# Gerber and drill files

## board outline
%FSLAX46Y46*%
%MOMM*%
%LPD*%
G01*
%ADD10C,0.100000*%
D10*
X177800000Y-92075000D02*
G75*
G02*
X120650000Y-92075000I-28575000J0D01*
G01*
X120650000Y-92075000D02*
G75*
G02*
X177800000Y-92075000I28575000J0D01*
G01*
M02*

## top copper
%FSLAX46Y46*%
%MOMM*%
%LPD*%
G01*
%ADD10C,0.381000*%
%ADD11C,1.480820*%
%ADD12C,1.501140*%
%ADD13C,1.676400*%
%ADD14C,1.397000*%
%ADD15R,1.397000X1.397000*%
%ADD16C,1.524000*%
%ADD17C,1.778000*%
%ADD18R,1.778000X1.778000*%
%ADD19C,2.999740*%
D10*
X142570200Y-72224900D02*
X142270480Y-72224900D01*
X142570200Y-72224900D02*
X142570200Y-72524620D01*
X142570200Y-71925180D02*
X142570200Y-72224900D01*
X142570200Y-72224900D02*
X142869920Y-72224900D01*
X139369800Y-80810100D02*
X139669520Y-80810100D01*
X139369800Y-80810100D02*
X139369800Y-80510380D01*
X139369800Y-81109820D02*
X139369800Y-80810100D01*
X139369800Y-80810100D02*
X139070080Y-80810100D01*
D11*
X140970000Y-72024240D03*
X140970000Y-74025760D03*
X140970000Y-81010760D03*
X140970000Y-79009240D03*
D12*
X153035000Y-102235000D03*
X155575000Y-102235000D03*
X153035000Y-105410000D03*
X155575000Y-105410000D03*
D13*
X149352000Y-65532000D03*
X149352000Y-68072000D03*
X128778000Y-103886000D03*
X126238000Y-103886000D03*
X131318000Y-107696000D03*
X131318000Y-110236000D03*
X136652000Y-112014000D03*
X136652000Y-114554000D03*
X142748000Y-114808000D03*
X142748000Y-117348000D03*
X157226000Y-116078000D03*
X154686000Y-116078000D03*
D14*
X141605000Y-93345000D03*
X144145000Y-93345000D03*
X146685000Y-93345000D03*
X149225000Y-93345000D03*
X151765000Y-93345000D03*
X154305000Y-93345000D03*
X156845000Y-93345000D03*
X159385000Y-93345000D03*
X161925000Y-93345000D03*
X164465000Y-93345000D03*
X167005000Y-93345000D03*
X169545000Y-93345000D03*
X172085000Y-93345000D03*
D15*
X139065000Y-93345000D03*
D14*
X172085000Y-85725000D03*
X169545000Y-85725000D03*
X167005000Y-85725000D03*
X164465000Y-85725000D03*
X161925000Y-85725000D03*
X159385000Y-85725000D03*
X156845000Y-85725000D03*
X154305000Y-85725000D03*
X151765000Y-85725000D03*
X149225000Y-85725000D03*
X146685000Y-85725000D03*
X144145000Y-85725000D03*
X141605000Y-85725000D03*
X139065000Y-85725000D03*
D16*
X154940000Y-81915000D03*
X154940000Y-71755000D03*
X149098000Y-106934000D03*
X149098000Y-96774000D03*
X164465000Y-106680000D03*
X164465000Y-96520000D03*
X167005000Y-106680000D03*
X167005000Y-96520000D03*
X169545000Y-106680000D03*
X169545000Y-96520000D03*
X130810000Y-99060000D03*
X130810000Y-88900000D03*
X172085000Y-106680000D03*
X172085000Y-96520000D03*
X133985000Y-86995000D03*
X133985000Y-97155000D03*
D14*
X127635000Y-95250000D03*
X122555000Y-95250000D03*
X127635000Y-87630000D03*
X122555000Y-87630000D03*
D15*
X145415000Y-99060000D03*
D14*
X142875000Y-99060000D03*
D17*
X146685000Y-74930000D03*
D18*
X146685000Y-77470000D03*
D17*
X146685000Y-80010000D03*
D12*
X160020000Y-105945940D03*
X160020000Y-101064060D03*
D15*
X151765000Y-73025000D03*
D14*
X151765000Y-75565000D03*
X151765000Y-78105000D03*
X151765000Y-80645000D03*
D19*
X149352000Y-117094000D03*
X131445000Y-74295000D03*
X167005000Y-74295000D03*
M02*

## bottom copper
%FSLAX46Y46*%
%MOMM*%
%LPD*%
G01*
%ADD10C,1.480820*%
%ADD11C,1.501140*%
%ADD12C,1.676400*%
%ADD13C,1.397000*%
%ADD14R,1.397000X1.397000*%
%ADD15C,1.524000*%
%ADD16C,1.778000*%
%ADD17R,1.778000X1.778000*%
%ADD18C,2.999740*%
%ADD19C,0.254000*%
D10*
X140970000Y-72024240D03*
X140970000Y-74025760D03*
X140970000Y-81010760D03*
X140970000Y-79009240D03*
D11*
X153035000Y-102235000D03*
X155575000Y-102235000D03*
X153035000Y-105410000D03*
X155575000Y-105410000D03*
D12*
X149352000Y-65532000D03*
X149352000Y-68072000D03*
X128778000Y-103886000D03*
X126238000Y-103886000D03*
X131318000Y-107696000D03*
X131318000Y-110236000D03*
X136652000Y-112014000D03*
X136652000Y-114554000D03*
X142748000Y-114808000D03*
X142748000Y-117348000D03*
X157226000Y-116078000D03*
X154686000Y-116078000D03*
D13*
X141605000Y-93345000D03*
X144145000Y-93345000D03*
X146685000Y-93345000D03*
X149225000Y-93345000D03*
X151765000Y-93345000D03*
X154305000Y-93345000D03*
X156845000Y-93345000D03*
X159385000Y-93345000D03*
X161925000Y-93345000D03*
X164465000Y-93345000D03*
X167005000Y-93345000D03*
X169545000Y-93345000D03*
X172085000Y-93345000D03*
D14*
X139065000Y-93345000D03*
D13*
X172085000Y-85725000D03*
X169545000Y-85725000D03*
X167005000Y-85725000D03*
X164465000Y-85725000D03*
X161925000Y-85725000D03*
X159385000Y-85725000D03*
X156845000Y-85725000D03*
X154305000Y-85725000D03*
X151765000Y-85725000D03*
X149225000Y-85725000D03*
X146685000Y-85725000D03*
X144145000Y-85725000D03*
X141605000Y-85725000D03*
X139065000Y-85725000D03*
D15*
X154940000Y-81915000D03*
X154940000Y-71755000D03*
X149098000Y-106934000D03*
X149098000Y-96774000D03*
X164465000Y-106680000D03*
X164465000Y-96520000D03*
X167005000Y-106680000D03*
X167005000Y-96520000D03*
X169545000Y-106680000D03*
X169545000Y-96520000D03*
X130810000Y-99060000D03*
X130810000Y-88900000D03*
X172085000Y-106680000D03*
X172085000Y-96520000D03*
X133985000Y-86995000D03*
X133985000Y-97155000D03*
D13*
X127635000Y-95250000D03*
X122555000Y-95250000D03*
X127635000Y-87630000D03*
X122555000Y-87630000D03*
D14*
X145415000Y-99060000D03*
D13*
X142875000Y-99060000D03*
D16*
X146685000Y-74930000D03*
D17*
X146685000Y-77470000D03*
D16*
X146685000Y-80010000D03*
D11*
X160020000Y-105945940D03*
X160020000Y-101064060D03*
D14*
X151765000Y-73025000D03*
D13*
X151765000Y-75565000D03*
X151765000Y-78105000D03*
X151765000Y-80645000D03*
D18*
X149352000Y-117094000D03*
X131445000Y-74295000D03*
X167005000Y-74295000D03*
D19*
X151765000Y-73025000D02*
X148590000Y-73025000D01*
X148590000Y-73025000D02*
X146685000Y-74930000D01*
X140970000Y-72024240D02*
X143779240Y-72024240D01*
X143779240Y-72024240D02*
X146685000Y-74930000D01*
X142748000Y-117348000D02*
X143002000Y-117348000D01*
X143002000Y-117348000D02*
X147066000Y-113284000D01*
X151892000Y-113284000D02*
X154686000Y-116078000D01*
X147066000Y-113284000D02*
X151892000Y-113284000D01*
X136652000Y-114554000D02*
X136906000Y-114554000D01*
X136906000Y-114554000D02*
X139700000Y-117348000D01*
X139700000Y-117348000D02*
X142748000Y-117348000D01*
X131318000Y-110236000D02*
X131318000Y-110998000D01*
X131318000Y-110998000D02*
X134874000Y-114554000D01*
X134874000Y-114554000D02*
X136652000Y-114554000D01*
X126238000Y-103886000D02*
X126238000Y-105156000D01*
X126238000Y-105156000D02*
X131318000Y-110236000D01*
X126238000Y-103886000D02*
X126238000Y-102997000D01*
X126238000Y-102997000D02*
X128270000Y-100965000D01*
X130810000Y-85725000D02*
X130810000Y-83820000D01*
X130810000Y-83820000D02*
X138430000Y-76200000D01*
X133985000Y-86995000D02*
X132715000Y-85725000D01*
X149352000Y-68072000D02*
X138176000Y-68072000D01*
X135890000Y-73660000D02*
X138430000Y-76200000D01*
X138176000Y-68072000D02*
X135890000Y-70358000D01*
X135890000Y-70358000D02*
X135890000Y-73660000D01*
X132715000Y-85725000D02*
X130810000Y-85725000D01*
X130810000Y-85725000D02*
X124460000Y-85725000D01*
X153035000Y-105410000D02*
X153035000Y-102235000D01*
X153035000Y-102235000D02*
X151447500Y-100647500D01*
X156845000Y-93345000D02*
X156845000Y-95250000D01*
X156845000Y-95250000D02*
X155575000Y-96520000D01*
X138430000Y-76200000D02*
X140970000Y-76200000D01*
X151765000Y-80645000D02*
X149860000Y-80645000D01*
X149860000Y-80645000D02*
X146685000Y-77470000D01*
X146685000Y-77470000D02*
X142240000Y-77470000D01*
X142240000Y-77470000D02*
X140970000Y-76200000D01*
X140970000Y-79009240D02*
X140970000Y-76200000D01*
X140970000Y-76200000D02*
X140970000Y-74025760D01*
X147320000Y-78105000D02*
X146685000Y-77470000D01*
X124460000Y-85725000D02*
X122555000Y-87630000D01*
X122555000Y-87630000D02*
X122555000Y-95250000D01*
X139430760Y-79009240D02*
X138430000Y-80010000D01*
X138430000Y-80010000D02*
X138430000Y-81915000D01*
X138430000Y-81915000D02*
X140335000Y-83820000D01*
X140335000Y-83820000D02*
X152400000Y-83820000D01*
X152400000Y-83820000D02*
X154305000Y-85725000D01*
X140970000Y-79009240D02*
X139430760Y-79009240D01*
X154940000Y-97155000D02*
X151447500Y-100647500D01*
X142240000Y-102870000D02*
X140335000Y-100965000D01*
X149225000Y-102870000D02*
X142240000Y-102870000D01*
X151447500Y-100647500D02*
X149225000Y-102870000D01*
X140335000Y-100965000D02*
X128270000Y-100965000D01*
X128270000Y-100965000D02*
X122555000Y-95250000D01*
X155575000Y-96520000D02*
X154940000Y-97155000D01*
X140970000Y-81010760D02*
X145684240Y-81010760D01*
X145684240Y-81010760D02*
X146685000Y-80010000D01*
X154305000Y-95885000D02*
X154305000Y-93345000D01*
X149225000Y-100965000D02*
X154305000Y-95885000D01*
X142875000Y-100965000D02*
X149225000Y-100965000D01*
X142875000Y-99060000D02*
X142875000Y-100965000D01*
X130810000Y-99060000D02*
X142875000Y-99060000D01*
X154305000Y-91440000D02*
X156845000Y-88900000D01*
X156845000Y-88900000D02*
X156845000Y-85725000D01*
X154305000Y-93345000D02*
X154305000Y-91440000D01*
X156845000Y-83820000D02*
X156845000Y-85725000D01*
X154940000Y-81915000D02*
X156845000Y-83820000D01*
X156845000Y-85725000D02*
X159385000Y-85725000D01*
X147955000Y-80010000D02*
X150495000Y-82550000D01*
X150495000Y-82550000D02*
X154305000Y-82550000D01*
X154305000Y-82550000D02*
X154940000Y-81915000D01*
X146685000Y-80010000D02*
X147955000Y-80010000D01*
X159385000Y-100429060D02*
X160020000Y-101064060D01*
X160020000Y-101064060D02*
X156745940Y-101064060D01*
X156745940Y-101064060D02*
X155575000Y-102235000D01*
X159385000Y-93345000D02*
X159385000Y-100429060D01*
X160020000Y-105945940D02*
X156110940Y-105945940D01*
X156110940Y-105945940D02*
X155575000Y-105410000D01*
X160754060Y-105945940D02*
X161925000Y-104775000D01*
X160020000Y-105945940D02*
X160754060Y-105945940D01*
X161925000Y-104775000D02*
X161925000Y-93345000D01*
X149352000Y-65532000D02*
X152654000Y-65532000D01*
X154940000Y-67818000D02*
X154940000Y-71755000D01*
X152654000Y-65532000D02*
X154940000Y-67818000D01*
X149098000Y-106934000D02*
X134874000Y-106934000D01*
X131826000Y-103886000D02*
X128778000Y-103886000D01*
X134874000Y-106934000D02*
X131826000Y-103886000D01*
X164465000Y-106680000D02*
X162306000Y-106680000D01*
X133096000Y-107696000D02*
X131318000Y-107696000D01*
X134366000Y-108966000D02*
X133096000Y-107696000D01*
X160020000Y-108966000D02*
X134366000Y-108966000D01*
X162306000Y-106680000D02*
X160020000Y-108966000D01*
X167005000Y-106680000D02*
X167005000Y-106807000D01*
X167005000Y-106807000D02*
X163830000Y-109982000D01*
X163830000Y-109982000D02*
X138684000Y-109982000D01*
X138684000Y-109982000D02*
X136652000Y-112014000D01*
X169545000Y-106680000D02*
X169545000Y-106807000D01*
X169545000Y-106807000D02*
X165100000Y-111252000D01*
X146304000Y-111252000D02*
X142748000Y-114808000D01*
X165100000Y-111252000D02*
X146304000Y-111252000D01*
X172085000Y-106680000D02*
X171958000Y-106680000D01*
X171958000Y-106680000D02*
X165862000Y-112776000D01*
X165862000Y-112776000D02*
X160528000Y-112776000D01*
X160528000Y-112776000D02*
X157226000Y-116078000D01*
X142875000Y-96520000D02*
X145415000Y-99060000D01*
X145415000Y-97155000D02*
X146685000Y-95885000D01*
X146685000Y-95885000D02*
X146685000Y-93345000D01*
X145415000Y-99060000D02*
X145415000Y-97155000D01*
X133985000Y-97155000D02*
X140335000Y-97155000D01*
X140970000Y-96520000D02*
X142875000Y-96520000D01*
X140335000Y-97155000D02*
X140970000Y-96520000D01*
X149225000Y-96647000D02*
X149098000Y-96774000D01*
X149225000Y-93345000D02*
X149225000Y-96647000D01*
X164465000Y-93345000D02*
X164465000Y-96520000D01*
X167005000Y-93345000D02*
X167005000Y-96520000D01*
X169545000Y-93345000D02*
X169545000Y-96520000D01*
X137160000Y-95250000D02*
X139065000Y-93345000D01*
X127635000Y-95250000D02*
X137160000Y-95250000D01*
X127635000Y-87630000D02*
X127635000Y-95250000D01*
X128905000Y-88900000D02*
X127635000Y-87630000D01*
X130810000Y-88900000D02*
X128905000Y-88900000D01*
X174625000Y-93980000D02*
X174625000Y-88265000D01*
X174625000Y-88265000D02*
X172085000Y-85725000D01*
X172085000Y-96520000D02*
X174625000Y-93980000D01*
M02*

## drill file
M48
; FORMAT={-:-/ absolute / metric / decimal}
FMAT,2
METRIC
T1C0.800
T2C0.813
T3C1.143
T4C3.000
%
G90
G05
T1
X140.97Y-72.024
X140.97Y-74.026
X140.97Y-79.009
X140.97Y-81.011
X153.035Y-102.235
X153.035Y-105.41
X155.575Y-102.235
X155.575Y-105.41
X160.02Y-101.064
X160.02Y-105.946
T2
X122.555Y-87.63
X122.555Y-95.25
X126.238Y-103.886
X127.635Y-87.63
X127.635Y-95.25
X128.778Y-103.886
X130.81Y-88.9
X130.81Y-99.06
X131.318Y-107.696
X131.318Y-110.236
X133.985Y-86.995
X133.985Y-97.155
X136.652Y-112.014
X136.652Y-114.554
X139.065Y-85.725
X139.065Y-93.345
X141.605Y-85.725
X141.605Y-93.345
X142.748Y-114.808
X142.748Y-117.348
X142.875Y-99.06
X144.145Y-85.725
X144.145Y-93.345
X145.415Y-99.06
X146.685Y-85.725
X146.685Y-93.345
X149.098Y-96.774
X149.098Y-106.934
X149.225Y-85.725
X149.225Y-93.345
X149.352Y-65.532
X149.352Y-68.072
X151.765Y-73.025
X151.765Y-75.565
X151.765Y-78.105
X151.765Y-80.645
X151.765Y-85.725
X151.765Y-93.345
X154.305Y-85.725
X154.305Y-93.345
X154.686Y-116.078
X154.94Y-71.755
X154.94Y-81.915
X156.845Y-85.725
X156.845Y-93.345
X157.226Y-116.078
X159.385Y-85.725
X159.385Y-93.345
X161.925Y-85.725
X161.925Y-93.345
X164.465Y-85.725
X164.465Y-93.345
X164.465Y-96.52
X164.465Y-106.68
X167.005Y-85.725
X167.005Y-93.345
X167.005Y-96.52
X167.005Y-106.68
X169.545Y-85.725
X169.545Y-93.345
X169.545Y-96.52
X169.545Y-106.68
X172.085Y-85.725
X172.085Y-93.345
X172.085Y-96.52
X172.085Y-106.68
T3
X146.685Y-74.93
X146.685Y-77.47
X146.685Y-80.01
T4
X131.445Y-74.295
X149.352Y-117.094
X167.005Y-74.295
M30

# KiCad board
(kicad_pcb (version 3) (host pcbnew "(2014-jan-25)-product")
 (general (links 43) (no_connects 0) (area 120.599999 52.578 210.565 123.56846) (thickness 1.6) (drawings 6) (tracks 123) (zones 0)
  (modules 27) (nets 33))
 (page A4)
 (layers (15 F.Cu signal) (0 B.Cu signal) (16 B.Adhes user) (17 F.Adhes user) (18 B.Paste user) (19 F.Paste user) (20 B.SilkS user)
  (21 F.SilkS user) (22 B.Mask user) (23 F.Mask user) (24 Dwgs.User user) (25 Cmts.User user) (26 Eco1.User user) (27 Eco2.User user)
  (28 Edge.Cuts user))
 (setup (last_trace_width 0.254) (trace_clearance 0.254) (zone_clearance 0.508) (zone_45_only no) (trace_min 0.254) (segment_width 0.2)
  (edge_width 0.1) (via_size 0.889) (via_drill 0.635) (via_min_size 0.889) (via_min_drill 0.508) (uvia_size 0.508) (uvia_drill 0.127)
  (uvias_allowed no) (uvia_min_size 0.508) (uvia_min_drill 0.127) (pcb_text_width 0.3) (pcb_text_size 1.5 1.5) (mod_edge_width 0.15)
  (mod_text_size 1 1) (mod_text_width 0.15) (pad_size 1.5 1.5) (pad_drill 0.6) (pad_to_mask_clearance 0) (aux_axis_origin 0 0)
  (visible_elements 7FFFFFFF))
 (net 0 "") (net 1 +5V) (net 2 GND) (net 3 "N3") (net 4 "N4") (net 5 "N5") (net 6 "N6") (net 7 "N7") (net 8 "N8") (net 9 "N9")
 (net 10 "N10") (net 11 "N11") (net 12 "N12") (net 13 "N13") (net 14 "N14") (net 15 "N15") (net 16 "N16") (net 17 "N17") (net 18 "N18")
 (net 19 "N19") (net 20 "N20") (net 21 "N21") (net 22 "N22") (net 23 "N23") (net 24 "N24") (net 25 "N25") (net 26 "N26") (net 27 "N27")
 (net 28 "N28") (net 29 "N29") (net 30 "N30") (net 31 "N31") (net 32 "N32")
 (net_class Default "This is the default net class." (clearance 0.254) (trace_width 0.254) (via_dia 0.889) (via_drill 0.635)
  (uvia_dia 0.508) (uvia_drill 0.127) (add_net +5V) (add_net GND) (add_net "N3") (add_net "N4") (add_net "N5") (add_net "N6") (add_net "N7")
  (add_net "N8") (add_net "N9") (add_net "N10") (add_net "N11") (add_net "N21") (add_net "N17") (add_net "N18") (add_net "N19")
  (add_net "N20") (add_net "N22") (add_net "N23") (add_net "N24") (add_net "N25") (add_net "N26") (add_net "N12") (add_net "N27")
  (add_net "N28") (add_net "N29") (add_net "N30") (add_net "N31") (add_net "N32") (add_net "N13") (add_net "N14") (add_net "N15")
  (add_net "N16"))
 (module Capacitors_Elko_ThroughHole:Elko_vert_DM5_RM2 (layer F.Cu) (at 140.97 73.025 270)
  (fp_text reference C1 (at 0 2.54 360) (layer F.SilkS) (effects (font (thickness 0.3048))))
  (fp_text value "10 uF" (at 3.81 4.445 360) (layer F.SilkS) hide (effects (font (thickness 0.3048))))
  (fp_line (start -0.8001 -1.6002) (end -0.8001 -1.30048) (layer F.Cu) (width 0.381))
  (fp_line (start -0.8001 -1.6002) (end -0.50038 -1.6002) (layer F.Cu) (width 0.381))
  (fp_line (start -1.09982 -1.6002) (end -0.8001 -1.6002) (layer F.Cu) (width 0.381))
  (fp_line (start -0.8001 -1.6002) (end -0.8001 -1.89992) (layer F.Cu) (width 0.381))
  (pad 1 thru_hole circle (at -1.00076 0 270) (size 1.48082 1.48082) (drill 0.8001) (layers *.Cu *.Mask F.SilkS) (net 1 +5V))
  (pad 2 thru_hole circle (at 1.00076 0 270) (size 1.48082 1.48082) (drill 0.8001) (layers *.Cu *.Mask F.SilkS) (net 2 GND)))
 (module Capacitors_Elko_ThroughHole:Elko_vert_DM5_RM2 (layer F.Cu) (at 140.97 80.01 90)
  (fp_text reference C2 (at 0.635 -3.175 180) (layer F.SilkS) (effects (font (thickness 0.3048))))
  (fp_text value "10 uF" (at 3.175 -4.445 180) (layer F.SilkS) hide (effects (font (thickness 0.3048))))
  (fp_line (start -0.8001 -1.6002) (end -0.8001 -1.30048) (layer F.Cu) (width 0.381))
  (fp_line (start -0.8001 -1.6002) (end -0.50038 -1.6002) (layer F.Cu) (width 0.381))
  (fp_line (start -1.09982 -1.6002) (end -0.8001 -1.6002) (layer F.Cu) (width 0.381))
  (fp_line (start -0.8001 -1.6002) (end -0.8001 -1.89992) (layer F.Cu) (width 0.381))
  (pad 1 thru_hole circle (at -1.00076 0 90) (size 1.48082 1.48082) (drill 0.8001) (layers *.Cu *.Mask F.SilkS) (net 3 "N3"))
  (pad 2 thru_hole circle (at 1.00076 0 90) (size 1.48082 1.48082) (drill 0.8001) (layers *.Cu *.Mask F.SilkS) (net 2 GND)))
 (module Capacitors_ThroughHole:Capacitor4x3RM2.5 (layer F.Cu) (at 153.035 102.235)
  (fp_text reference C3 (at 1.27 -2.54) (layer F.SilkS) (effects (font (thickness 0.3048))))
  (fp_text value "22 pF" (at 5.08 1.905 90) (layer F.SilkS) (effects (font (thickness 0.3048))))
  (pad 1 thru_hole circle (at 0 0) (size 1.50114 1.50114) (drill 0.8001) (layers *.Cu *.Mask F.SilkS) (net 2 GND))
  (pad 2 thru_hole circle (at 2.54 0) (size 1.50114 1.50114) (drill 0.8001) (layers *.Cu *.Mask F.SilkS) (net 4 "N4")))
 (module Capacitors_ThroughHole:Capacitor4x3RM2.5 (layer F.Cu) (at 153.035 105.41)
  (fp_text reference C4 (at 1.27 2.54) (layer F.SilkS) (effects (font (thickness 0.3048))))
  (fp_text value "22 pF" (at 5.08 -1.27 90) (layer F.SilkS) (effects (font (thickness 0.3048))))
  (pad 1 thru_hole circle (at 0 0) (size 1.50114 1.50114) (drill 0.8001) (layers *.Cu *.Mask F.SilkS) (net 2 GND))
  (pad 2 thru_hole circle (at 2.54 0) (size 1.50114 1.50114) (drill 0.8001) (layers *.Cu *.Mask F.SilkS) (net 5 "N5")))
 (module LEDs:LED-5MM (layer F.Cu) (at 149.352 66.802 270)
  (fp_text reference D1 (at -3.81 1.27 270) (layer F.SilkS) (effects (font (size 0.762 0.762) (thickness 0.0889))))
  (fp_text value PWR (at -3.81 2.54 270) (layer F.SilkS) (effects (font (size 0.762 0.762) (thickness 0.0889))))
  (pad 1 thru_hole circle (at -1.27 0 270) (size 1.6764 1.6764) (drill 0.8128) (layers *.Cu *.Mask F.SilkS) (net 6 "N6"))
  (pad 2 thru_hole circle (at 1.27 0 270) (size 1.6764 1.6764) (drill 0.8128) (layers *.Cu *.Mask F.SilkS) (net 2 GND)))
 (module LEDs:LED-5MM (layer F.Cu) (at 127.508 103.886 180)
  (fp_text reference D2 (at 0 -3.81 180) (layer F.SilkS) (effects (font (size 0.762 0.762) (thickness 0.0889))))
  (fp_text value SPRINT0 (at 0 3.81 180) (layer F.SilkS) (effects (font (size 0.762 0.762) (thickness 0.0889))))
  (pad 1 thru_hole circle (at -1.27 0 180) (size 1.6764 1.6764) (drill 0.8128) (layers *.Cu *.Mask F.SilkS) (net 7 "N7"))
  (pad 2 thru_hole circle (at 1.27 0 180) (size 1.6764 1.6764) (drill 0.8128) (layers *.Cu *.Mask F.SilkS) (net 2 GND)))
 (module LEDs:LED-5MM (layer F.Cu) (at 131.318 108.966 270)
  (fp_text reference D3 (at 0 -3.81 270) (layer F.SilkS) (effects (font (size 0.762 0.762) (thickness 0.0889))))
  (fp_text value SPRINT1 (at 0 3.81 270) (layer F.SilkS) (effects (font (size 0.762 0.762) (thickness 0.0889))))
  (pad 1 thru_hole circle (at -1.27 0 270) (size 1.6764 1.6764) (drill 0.8128) (layers *.Cu *.Mask F.SilkS) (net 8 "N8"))
  (pad 2 thru_hole circle (at 1.27 0 270) (size 1.6764 1.6764) (drill 0.8128) (layers *.Cu *.Mask F.SilkS) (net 2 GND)))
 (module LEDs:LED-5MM (layer F.Cu) (at 136.652 113.284 270)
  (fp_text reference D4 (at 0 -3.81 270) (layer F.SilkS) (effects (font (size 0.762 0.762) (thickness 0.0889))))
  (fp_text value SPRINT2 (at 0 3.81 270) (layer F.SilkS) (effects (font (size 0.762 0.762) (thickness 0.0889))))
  (pad 1 thru_hole circle (at -1.27 0 270) (size 1.6764 1.6764) (drill 0.8128) (layers *.Cu *.Mask F.SilkS) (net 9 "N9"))
  (pad 2 thru_hole circle (at 1.27 0 270) (size 1.6764 1.6764) (drill 0.8128) (layers *.Cu *.Mask F.SilkS) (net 2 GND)))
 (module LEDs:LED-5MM (layer F.Cu) (at 142.748 116.078 270)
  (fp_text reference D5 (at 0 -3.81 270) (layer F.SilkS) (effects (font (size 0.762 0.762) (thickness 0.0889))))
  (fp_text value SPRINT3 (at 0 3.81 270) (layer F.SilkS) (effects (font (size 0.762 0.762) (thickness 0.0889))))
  (pad 1 thru_hole circle (at -1.27 0 270) (size 1.6764 1.6764) (drill 0.8128) (layers *.Cu *.Mask F.SilkS) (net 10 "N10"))
  (pad 2 thru_hole circle (at 1.27 0 270) (size 1.6764 1.6764) (drill 0.8128) (layers *.Cu *.Mask F.SilkS) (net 2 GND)))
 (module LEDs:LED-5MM (layer F.Cu) (at 155.956 116.078 180)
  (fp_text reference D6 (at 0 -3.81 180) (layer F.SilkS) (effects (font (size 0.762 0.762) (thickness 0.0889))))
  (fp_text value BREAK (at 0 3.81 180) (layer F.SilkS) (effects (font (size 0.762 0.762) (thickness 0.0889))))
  (pad 1 thru_hole circle (at -1.27 0 180) (size 1.6764 1.6764) (drill 0.8128) (layers *.Cu *.Mask F.SilkS) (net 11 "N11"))
  (pad 2 thru_hole circle (at 1.27 0 180) (size 1.6764 1.6764) (drill 0.8128) (layers *.Cu *.Mask F.SilkS) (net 2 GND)))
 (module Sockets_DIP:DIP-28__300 (layer F.Cu) (at 155.575 89.535)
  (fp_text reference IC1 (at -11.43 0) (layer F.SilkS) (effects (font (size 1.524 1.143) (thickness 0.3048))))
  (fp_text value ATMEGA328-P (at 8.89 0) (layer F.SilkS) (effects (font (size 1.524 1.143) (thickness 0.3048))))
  (pad 2 thru_hole circle (at -13.97 3.81) (size 1.397 1.397) (drill 0.8128) (layers *.Cu *.Mask F.SilkS) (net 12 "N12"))
  (pad 3 thru_hole circle (at -11.43 3.81) (size 1.397 1.397) (drill 0.8128) (layers *.Cu *.Mask F.SilkS) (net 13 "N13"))
  (pad 4 thru_hole circle (at -8.89 3.81) (size 1.397 1.397) (drill 0.8128) (layers *.Cu *.Mask F.SilkS) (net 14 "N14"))
  (pad 5 thru_hole circle (at -6.35 3.81) (size 1.397 1.397) (drill 0.8128) (layers *.Cu *.Mask F.SilkS) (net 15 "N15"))
  (pad 6 thru_hole circle (at -3.81 3.81) (size 1.397 1.397) (drill 0.8128) (layers *.Cu *.Mask F.SilkS) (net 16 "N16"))
  (pad 7 thru_hole circle (at -1.27 3.81) (size 1.397 1.397) (drill 0.8128) (layers *.Cu *.Mask F.SilkS) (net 3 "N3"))
  (pad 8 thru_hole circle (at 1.27 3.81) (size 1.397 1.397) (drill 0.8128) (layers *.Cu *.Mask F.SilkS) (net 2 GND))
  (pad 9 thru_hole circle (at 3.81 3.81) (size 1.397 1.397) (drill 0.8128) (layers *.Cu *.Mask F.SilkS) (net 4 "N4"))
  (pad 10 thru_hole circle (at 6.35 3.81) (size 1.397 1.397) (drill 0.8128) (layers *.Cu *.Mask F.SilkS) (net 5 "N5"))
  (pad 11 thru_hole circle (at 8.89 3.81) (size 1.397 1.397) (drill 0.8128) (layers *.Cu *.Mask F.SilkS) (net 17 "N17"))
  (pad 12 thru_hole circle (at 11.43 3.81) (size 1.397 1.397) (drill 0.8128) (layers *.Cu *.Mask F.SilkS) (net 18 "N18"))
  (pad 13 thru_hole circle (at 13.97 3.81) (size 1.397 1.397) (drill 0.8128) (layers *.Cu *.Mask F.SilkS) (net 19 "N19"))
  (pad 14 thru_hole circle (at 16.51 3.81) (size 1.397 1.397) (drill 0.8128) (layers *.Cu *.Mask F.SilkS) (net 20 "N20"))
  (pad 1 thru_hole rect (at -16.51 3.81) (size 1.397 1.397) (drill 0.8128) (layers *.Cu *.Mask F.SilkS) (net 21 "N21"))
  (pad 15 thru_hole circle (at 16.51 -3.81) (size 1.397 1.397) (drill 0.8128) (layers *.Cu *.Mask F.SilkS) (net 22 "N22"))
  (pad 16 thru_hole circle (at 13.97 -3.81) (size 1.397 1.397) (drill 0.8128) (layers *.Cu *.Mask F.SilkS) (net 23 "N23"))
  (pad 17 thru_hole circle (at 11.43 -3.81) (size 1.397 1.397) (drill 0.8128) (layers *.Cu *.Mask F.SilkS) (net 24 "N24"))
  (pad 18 thru_hole circle (at 8.89 -3.81) (size 1.397 1.397) (drill 0.8128) (layers *.Cu *.Mask F.SilkS) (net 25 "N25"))
  (pad 19 thru_hole circle (at 6.35 -3.81) (size 1.397 1.397) (drill 0.8128) (layers *.Cu *.Mask F.SilkS) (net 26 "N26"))
  (pad 20 thru_hole circle (at 3.81 -3.81) (size 1.397 1.397) (drill 0.8128) (layers *.Cu *.Mask F.SilkS) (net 3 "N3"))
  (pad 21 thru_hole circle (at 1.27 -3.81) (size 1.397 1.397) (drill 0.8128) (layers *.Cu *.Mask F.SilkS) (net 3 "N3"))
  (pad 22 thru_hole circle (at -1.27 -3.81) (size 1.397 1.397) (drill 0.8128) (layers *.Cu *.Mask F.SilkS) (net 2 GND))
  (pad 23 thru_hole circle (at -3.81 -3.81) (size 1.397 1.397) (drill 0.8128) (layers *.Cu *.Mask F.SilkS) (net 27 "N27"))
  (pad 24 thru_hole circle (at -6.35 -3.81) (size 1.397 1.397) (drill 0.8128) (layers *.Cu *.Mask F.SilkS) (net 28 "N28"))
  (pad 25 thru_hole circle (at -8.89 -3.81) (size 1.397 1.397) (drill 0.8128) (layers *.Cu *.Mask F.SilkS) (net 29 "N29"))
  (pad 26 thru_hole circle (at -11.43 -3.81) (size 1.397 1.397) (drill 0.8128) (layers *.Cu *.Mask F.SilkS) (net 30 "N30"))
  (pad 27 thru_hole circle (at -13.97 -3.81) (size 1.397 1.397) (drill 0.8128) (layers *.Cu *.Mask F.SilkS) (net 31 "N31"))
  (pad 28 thru_hole circle (at -16.51 -3.81) (size 1.397 1.397) (drill 0.8128) (layers *.Cu *.Mask F.SilkS) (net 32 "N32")))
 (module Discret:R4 (layer F.Cu) (at 154.94 76.835 90) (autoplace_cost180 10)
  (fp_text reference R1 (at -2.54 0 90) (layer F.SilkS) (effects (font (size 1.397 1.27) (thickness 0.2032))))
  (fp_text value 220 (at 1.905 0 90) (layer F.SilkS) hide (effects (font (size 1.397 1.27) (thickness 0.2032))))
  (pad 1 thru_hole circle (at -5.08 0 90) (size 1.524 1.524) (drill 0.8128) (layers *.Cu *.Mask F.SilkS) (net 3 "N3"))
  (pad 2 thru_hole circle (at 5.08 0 90) (size 1.524 1.524) (drill 0.8128) (layers *.Cu *.Mask F.SilkS) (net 6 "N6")))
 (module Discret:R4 (layer F.Cu) (at 149.098 101.854 90) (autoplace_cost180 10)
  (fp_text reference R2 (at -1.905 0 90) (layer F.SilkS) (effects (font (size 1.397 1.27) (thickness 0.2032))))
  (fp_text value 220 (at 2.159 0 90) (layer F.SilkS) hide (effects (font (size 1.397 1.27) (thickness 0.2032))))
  (pad 1 thru_hole circle (at -5.08 0 90) (size 1.524 1.524) (drill 0.8128) (layers *.Cu *.Mask F.SilkS) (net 7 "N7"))
  (pad 2 thru_hole circle (at 5.08 0 90) (size 1.524 1.524) (drill 0.8128) (layers *.Cu *.Mask F.SilkS) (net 15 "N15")))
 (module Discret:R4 (layer F.Cu) (at 164.465 101.6 90) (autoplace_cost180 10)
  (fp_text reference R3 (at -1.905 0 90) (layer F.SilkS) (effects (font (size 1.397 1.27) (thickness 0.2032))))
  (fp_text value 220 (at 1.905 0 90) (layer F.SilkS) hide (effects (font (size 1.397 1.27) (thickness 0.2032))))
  (pad 1 thru_hole circle (at -5.08 0 90) (size 1.524 1.524) (drill 0.8128) (layers *.Cu *.Mask F.SilkS) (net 8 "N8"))
  (pad 2 thru_hole circle (at 5.08 0 90) (size 1.524 1.524) (drill 0.8128) (layers *.Cu *.Mask F.SilkS) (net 17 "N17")))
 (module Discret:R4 (layer F.Cu) (at 167.005 101.6 90) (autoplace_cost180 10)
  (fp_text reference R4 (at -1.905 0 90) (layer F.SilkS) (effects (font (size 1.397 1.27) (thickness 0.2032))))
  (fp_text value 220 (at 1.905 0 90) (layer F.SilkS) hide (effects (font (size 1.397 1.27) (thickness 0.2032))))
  (pad 1 thru_hole circle (at -5.08 0 90) (size 1.524 1.524) (drill 0.8128) (layers *.Cu *.Mask F.SilkS) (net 9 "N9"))
  (pad 2 thru_hole circle (at 5.08 0 90) (size 1.524 1.524) (drill 0.8128) (layers *.Cu *.Mask F.SilkS) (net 18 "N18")))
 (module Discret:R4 (layer F.Cu) (at 169.545 101.6 90) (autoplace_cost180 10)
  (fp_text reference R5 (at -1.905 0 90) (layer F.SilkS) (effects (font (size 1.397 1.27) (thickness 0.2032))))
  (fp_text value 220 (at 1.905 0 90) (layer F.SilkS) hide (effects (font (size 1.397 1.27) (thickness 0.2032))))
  (pad 1 thru_hole circle (at -5.08 0 90) (size 1.524 1.524) (drill 0.8128) (layers *.Cu *.Mask F.SilkS) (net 10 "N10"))
  (pad 2 thru_hole circle (at 5.08 0 90) (size 1.524 1.524) (drill 0.8128) (layers *.Cu *.Mask F.SilkS) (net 19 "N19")))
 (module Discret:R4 (layer F.Cu) (at 130.81 93.98 90) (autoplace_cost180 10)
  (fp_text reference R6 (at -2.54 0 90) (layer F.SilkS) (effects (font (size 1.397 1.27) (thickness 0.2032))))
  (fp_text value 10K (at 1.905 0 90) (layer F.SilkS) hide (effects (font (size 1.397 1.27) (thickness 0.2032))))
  (pad 1 thru_hole circle (at -5.08 0 90) (size 1.524 1.524) (drill 0.8128) (layers *.Cu *.Mask F.SilkS) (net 3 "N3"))
  (pad 2 thru_hole circle (at 5.08 0 90) (size 1.524 1.524) (drill 0.8128) (layers *.Cu *.Mask F.SilkS) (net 21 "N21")))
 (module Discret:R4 (layer F.Cu) (at 172.085 101.6 90) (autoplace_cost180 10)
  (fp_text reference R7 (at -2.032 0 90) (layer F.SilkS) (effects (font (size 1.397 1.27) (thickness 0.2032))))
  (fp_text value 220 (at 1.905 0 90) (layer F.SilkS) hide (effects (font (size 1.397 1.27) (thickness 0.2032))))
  (pad 1 thru_hole circle (at -5.08 0 90) (size 1.524 1.524) (drill 0.8128) (layers *.Cu *.Mask F.SilkS) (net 11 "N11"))
  (pad 2 thru_hole circle (at 5.08 0 90) (size 1.524 1.524) (drill 0.8128) (layers *.Cu *.Mask F.SilkS) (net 22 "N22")))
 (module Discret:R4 (layer F.Cu) (at 133.985 92.075 270) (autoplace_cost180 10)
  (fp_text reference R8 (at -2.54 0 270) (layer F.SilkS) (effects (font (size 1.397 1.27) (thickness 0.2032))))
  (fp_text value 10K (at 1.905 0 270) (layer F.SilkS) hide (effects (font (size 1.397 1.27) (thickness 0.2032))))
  (pad 1 thru_hole circle (at -5.08 0 270) (size 1.524 1.524) (drill 0.8128) (layers *.Cu *.Mask F.SilkS) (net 2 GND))
  (pad 2 thru_hole circle (at 5.08 0 270) (size 1.524 1.524) (drill 0.8128) (layers *.Cu *.Mask F.SilkS) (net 14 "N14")))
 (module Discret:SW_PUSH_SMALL (layer F.Cu) (at 125.095 91.44 270)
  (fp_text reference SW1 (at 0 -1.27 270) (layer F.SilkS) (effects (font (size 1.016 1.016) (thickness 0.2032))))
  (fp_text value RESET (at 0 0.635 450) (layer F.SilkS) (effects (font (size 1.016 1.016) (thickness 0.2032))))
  (pad 1 thru_hole circle (at 3.81 -2.54 270) (size 1.397 1.397) (drill 0.8128) (layers *.Cu *.Mask F.SilkS) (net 21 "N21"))
  (pad 2 thru_hole circle (at 3.81 2.54 270) (size 1.397 1.397) (drill 0.8128) (layers *.Cu *.Mask F.SilkS) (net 2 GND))
  (pad 1 thru_hole circle (at -3.81 -2.54 270) (size 1.397 1.397) (drill 0.8128) (layers *.Cu *.Mask F.SilkS) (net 21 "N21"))
  (pad 2 thru_hole circle (at -3.81 2.54 270) (size 1.397 1.397) (drill 0.8128) (layers *.Cu *.Mask F.SilkS) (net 2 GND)))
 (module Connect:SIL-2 (layer F.Cu) (at 144.145 99.06 180)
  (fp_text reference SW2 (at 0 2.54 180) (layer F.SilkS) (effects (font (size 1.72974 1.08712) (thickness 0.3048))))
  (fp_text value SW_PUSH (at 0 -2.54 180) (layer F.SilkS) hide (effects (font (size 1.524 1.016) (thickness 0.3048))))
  (pad 1 thru_hole rect (at -1.27 0 180) (size 1.397 1.397) (drill 0.8128) (layers *.Cu *.Mask F.SilkS) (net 14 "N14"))
  (pad 2 thru_hole circle (at 1.27 0 180) (size 1.397 1.397) (drill 0.8128) (layers *.Cu *.Mask F.SilkS) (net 3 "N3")))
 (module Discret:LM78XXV (layer F.Cu) (at 146.685 77.47)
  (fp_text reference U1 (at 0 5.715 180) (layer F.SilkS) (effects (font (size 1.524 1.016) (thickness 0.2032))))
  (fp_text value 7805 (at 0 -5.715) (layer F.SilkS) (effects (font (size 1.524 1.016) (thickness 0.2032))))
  (pad VI thru_hole circle (at 0 -2.54) (size 1.778 1.778) (drill 1.143) (layers *.Cu *.Mask F.SilkS) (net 1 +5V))
  (pad GND thru_hole rect (at 0 0) (size 1.778 1.778) (drill 1.143) (layers *.Cu *.Mask F.SilkS) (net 2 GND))
  (pad VO thru_hole circle (at 0 2.54) (size 1.778 1.778) (drill 1.143) (layers *.Cu *.Mask F.SilkS) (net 3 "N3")))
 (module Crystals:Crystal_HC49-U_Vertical (layer F.Cu) (at 160.02 103.505 90)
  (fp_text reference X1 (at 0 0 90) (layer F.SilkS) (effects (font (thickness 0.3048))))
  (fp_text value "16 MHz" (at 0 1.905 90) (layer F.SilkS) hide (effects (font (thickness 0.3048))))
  (pad 1 thru_hole circle (at -2.44094 0 90) (size 1.50114 1.50114) (drill 0.8001) (layers *.Cu *.Mask F.SilkS) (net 5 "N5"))
  (pad 2 thru_hole circle (at 2.44094 0 90) (size 1.50114 1.50114) (drill 0.8001) (layers *.Cu *.Mask F.SilkS) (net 4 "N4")))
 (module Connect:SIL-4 (layer F.Cu) (at 151.765 76.835 270)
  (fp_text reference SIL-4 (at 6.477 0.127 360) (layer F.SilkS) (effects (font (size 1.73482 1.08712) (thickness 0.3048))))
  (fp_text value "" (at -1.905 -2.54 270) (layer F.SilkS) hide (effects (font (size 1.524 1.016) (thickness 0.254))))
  (pad 1 thru_hole rect (at -3.81 0 270) (size 1.397 1.397) (drill 0.8128) (layers *.Cu *.Mask F.SilkS))
  (pad 2 thru_hole circle (at -1.27 0 270) (size 1.397 1.397) (drill 0.8128) (layers *.Cu *.Mask F.SilkS))
  (pad 3 thru_hole circle (at 1.27 0 270) (size 1.397 1.397) (drill 0.8128) (layers *.Cu *.Mask F.SilkS))
  (pad 4 thru_hole circle (at 3.81 0 270) (size 1.397 1.397) (drill 0.8128) (layers *.Cu *.Mask F.SilkS)))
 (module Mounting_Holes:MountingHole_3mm (layer F.Cu) (at 149.352 117.094)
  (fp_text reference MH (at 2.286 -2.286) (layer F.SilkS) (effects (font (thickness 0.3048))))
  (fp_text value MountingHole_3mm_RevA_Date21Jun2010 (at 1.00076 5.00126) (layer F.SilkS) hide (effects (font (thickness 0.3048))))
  (pad 1 thru_hole circle (at 0 0) (size 2.99974 2.99974) (drill 2.99974) (layers)))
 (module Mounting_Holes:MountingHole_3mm (layer F.Cu) (at 131.445 74.295)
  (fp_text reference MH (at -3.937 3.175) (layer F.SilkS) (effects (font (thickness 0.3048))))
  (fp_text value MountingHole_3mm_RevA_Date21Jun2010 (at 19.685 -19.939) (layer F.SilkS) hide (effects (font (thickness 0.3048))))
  (pad 1 thru_hole circle (at 0 0) (size 2.99974 2.99974) (drill 2.99974) (layers)))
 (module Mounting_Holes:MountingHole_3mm (layer F.Cu) (at 167.005 74.295)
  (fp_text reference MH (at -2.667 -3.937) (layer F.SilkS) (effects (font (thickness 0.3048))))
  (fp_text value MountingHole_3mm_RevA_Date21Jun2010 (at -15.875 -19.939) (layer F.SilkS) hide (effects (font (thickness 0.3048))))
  (pad 1 thru_hole circle (at 0 0) (size 2.99974 2.99974) (drill 2.99974) (layers)))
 (gr_circle (center 149.225 92.075) (end 149.225 120.65) (layer Edge.Cuts) (width 0.1))
 (segment (start 151.765 73.025) (end 148.59 73.025) (width 0.254) (layer B.Cu) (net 1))
 (segment (start 148.59 73.025) (end 146.685 74.93) (width 0.254) (layer B.Cu) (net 1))
 (segment (start 140.97 72.02424) (end 143.77924 72.02424) (width 0.254) (layer B.Cu) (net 1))
 (segment (start 143.77924 72.02424) (end 146.685 74.93) (width 0.254) (layer B.Cu) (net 1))
 (segment (start 142.748 117.348) (end 143.002 117.348) (width 0.254) (layer B.Cu) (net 2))
 (segment (start 143.002 117.348) (end 147.066 113.284) (width 0.254) (layer B.Cu) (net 2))
 (segment (start 151.892 113.284) (end 154.686 116.078) (width 0.254) (layer B.Cu) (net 2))
 (segment (start 147.066 113.284) (end 151.892 113.284) (width 0.254) (layer B.Cu) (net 2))
 (segment (start 136.652 114.554) (end 136.906 114.554) (width 0.254) (layer B.Cu) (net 2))
 (segment (start 136.906 114.554) (end 139.7 117.348) (width 0.254) (layer B.Cu) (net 2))
 (segment (start 139.7 117.348) (end 142.748 117.348) (width 0.254) (layer B.Cu) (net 2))
 (segment (start 131.318 110.236) (end 131.318 110.998) (width 0.254) (layer B.Cu) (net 2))
 (segment (start 131.318 110.998) (end 134.874 114.554) (width 0.254) (layer B.Cu) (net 2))
 (segment (start 134.874 114.554) (end 136.652 114.554) (width 0.254) (layer B.Cu) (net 2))
 (segment (start 126.238 103.886) (end 126.238 105.156) (width 0.254) (layer B.Cu) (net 2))
 (segment (start 126.238 105.156) (end 131.318 110.236) (width 0.254) (layer B.Cu) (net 2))
 (segment (start 126.238 103.886) (end 126.238 102.997) (width 0.254) (layer B.Cu) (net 2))
 (segment (start 126.238 102.997) (end 128.27 100.965) (width 0.254) (layer B.Cu) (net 2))
 (segment (start 130.81 85.725) (end 130.81 83.82) (width 0.254) (layer B.Cu) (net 2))
 (segment (start 130.81 83.82) (end 138.43 76.2) (width 0.254) (layer B.Cu) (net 2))
 (segment (start 133.985 86.995) (end 132.715 85.725) (width 0.254) (layer B.Cu) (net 2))
 (segment (start 149.352 68.072) (end 138.176 68.072) (width 0.254) (layer B.Cu) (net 2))
 (segment (start 135.89 73.66) (end 138.43 76.2) (width 0.254) (layer B.Cu) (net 2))
 (segment (start 138.176 68.072) (end 135.89 70.358) (width 0.254) (layer B.Cu) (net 2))
 (segment (start 135.89 70.358) (end 135.89 73.66) (width 0.254) (layer B.Cu) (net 2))
 (segment (start 132.715 85.725) (end 130.81 85.725) (width 0.254) (layer B.Cu) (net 2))
 (segment (start 130.81 85.725) (end 124.46 85.725) (width 0.254) (layer B.Cu) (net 2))
 (segment (start 153.035 105.41) (end 153.035 102.235) (width 0.254) (layer B.Cu) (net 2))
 (segment (start 153.035 102.235) (end 151.4475 100.6475) (width 0.254) (layer B.Cu) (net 2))
 (segment (start 156.845 93.345) (end 156.845 95.25) (width 0.254) (layer B.Cu) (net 2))
 (segment (start 156.845 95.25) (end 155.575 96.52) (width 0.254) (layer B.Cu) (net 2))
 (segment (start 138.43 76.2) (end 140.97 76.2) (width 0.254) (layer B.Cu) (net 2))
 (segment (start 151.765 80.645) (end 149.86 80.645) (width 0.254) (layer B.Cu) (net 2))
 (segment (start 149.86 80.645) (end 146.685 77.47) (width 0.254) (layer B.Cu) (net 2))
 (segment (start 146.685 77.47) (end 142.24 77.47) (width 0.254) (layer B.Cu) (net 2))
 (segment (start 142.24 77.47) (end 140.97 76.2) (width 0.254) (layer B.Cu) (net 2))
 (segment (start 140.97 79.00924) (end 140.97 76.2) (width 0.254) (layer B.Cu) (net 2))
 (segment (start 140.97 76.2) (end 140.97 74.02576) (width 0.254) (layer B.Cu) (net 2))
 (segment (start 147.32 78.105) (end 146.685 77.47) (width 0.254) (layer B.Cu) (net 2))
 (segment (start 124.46 85.725) (end 122.555 87.63) (width 0.254) (layer B.Cu) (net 2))
 (segment (start 122.555 87.63) (end 122.555 95.25) (width 0.254) (layer B.Cu) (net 2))
 (segment (start 139.43076 79.00924) (end 138.43 80.01) (width 0.254) (layer B.Cu) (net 2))
 (segment (start 138.43 80.01) (end 138.43 81.915) (width 0.254) (layer B.Cu) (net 2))
 (segment (start 138.43 81.915) (end 140.335 83.82) (width 0.254) (layer B.Cu) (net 2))
 (segment (start 140.335 83.82) (end 152.4 83.82) (width 0.254) (layer B.Cu) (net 2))
 (segment (start 152.4 83.82) (end 154.305 85.725) (width 0.254) (layer B.Cu) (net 2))
 (segment (start 140.97 79.00924) (end 139.43076 79.00924) (width 0.254) (layer B.Cu) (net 2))
 (segment (start 154.94 97.155) (end 151.4475 100.6475) (width 0.254) (layer B.Cu) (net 2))
 (segment (start 142.24 102.87) (end 140.335 100.965) (width 0.254) (layer B.Cu) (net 2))
 (segment (start 149.225 102.87) (end 142.24 102.87) (width 0.254) (layer B.Cu) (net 2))
 (segment (start 151.4475 100.6475) (end 149.225 102.87) (width 0.254) (layer B.Cu) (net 2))
 (segment (start 140.335 100.965) (end 128.27 100.965) (width 0.254) (layer B.Cu) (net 2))
 (segment (start 128.27 100.965) (end 122.555 95.25) (width 0.254) (layer B.Cu) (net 2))
 (segment (start 155.575 96.52) (end 154.94 97.155) (width 0.254) (layer B.Cu) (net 2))
 (segment (start 140.97 81.01076) (end 145.68424 81.01076) (width 0.254) (layer B.Cu) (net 3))
 (segment (start 145.68424 81.01076) (end 146.685 80.01) (width 0.254) (layer B.Cu) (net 3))
 (segment (start 154.305 95.885) (end 154.305 93.345) (width 0.254) (layer B.Cu) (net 3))
 (segment (start 149.225 100.965) (end 154.305 95.885) (width 0.254) (layer B.Cu) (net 3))
 (segment (start 142.875 100.965) (end 149.225 100.965) (width 0.254) (layer B.Cu) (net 3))
 (segment (start 142.875 99.06) (end 142.875 100.965) (width 0.254) (layer B.Cu) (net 3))
 (segment (start 130.81 99.06) (end 142.875 99.06) (width 0.254) (layer B.Cu) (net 3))
 (segment (start 154.305 91.44) (end 156.845 88.9) (width 0.254) (layer B.Cu) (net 3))
 (segment (start 156.845 88.9) (end 156.845 85.725) (width 0.254) (layer B.Cu) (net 3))
 (segment (start 154.305 93.345) (end 154.305 91.44) (width 0.254) (layer B.Cu) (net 3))
 (segment (start 156.845 83.82) (end 156.845 85.725) (width 0.254) (layer B.Cu) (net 3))
 (segment (start 154.94 81.915) (end 156.845 83.82) (width 0.254) (layer B.Cu) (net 3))
 (segment (start 156.845 85.725) (end 159.385 85.725) (width 0.254) (layer B.Cu) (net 3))
 (segment (start 147.955 80.01) (end 150.495 82.55) (width 0.254) (layer B.Cu) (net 3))
 (segment (start 150.495 82.55) (end 154.305 82.55) (width 0.254) (layer B.Cu) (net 3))
 (segment (start 154.305 82.55) (end 154.94 81.915) (width 0.254) (layer B.Cu) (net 3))
 (segment (start 146.685 80.01) (end 147.955 80.01) (width 0.254) (layer B.Cu) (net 3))
 (segment (start 159.385 100.42906) (end 160.02 101.06406) (width 0.254) (layer B.Cu) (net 4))
 (segment (start 160.02 101.06406) (end 156.74594 101.06406) (width 0.254) (layer B.Cu) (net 4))
 (segment (start 156.74594 101.06406) (end 155.575 102.235) (width 0.254) (layer B.Cu) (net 4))
 (segment (start 159.385 93.345) (end 159.385 100.42906) (width 0.254) (layer B.Cu) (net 4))
 (segment (start 160.02 105.94594) (end 156.11094 105.94594) (width 0.254) (layer B.Cu) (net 5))
 (segment (start 156.11094 105.94594) (end 155.575 105.41) (width 0.254) (layer B.Cu) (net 5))
 (segment (start 160.75406 105.94594) (end 161.925 104.775) (width 0.254) (layer B.Cu) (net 5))
 (segment (start 160.02 105.94594) (end 160.75406 105.94594) (width 0.254) (layer B.Cu) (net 5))
 (segment (start 161.925 104.775) (end 161.925 93.345) (width 0.254) (layer B.Cu) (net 5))
 (segment (start 149.352 65.532) (end 152.654 65.532) (width 0.254) (layer B.Cu) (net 6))
 (segment (start 154.94 67.818) (end 154.94 71.755) (width 0.254) (layer B.Cu) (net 6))
 (segment (start 152.654 65.532) (end 154.94 67.818) (width 0.254) (layer B.Cu) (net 6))
 (segment (start 149.098 106.934) (end 134.874 106.934) (width 0.254) (layer B.Cu) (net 7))
 (segment (start 131.826 103.886) (end 128.778 103.886) (width 0.254) (layer B.Cu) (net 7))
 (segment (start 134.874 106.934) (end 131.826 103.886) (width 0.254) (layer B.Cu) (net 7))
 (segment (start 164.465 106.68) (end 162.306 106.68) (width 0.254) (layer B.Cu) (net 8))
 (segment (start 133.096 107.696) (end 131.318 107.696) (width 0.254) (layer B.Cu) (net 8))
 (segment (start 134.366 108.966) (end 133.096 107.696) (width 0.254) (layer B.Cu) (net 8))
 (segment (start 160.02 108.966) (end 134.366 108.966) (width 0.254) (layer B.Cu) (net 8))
 (segment (start 162.306 106.68) (end 160.02 108.966) (width 0.254) (layer B.Cu) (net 8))
 (segment (start 167.005 106.68) (end 167.005 106.807) (width 0.254) (layer B.Cu) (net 9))
 (segment (start 167.005 106.807) (end 163.83 109.982) (width 0.254) (layer B.Cu) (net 9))
 (segment (start 163.83 109.982) (end 138.684 109.982) (width 0.254) (layer B.Cu) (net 9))
 (segment (start 138.684 109.982) (end 136.652 112.014) (width 0.254) (layer B.Cu) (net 9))
 (segment (start 169.545 106.68) (end 169.545 106.807) (width 0.254) (layer B.Cu) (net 10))
 (segment (start 169.545 106.807) (end 165.1 111.252) (width 0.254) (layer B.Cu) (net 10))
 (segment (start 146.304 111.252) (end 142.748 114.808) (width 0.254) (layer B.Cu) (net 10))
 (segment (start 165.1 111.252) (end 146.304 111.252) (width 0.254) (layer B.Cu) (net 10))
 (segment (start 172.085 106.68) (end 171.958 106.68) (width 0.254) (layer B.Cu) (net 11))
 (segment (start 171.958 106.68) (end 165.862 112.776) (width 0.254) (layer B.Cu) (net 11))
 (segment (start 165.862 112.776) (end 160.528 112.776) (width 0.254) (layer B.Cu) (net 11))
 (segment (start 160.528 112.776) (end 157.226 116.078) (width 0.254) (layer B.Cu) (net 11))
 (segment (start 142.875 96.52) (end 145.415 99.06) (width 0.254) (layer B.Cu) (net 14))
 (segment (start 145.415 97.155) (end 146.685 95.885) (width 0.254) (layer B.Cu) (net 14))
 (segment (start 146.685 95.885) (end 146.685 93.345) (width 0.254) (layer B.Cu) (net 14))
 (segment (start 145.415 99.06) (end 145.415 97.155) (width 0.254) (layer B.Cu) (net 14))
 (segment (start 133.985 97.155) (end 140.335 97.155) (width 0.254) (layer B.Cu) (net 14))
 (segment (start 140.97 96.52) (end 142.875 96.52) (width 0.254) (layer B.Cu) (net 14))
 (segment (start 140.335 97.155) (end 140.97 96.52) (width 0.254) (layer B.Cu) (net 14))
 (segment (start 149.225 96.647) (end 149.098 96.774) (width 0.254) (layer B.Cu) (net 15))
 (segment (start 149.225 93.345) (end 149.225 96.647) (width 0.254) (layer B.Cu) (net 15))
 (segment (start 164.465 93.345) (end 164.465 96.52) (width 0.254) (layer B.Cu) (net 17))
 (segment (start 167.005 93.345) (end 167.005 96.52) (width 0.254) (layer B.Cu) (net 18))
 (segment (start 169.545 93.345) (end 169.545 96.52) (width 0.254) (layer B.Cu) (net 19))
 (segment (start 137.16 95.25) (end 139.065 93.345) (width 0.254) (layer B.Cu) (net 21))
 (segment (start 127.635 95.25) (end 137.16 95.25) (width 0.254) (layer B.Cu) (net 21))
 (segment (start 127.635 87.63) (end 127.635 95.25) (width 0.254) (layer B.Cu) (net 21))
 (segment (start 128.905 88.9) (end 127.635 87.63) (width 0.254) (layer B.Cu) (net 21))
 (segment (start 130.81 88.9) (end 128.905 88.9) (width 0.254) (layer B.Cu) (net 21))
 (segment (start 174.625 93.98) (end 174.625 88.265) (width 0.254) (layer B.Cu) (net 22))
 (segment (start 174.625 88.265) (end 172.085 85.725) (width 0.254) (layer B.Cu) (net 22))
 (segment (start 172.085 96.52) (end 174.625 93.98) (width 0.254) (layer B.Cu) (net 22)))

